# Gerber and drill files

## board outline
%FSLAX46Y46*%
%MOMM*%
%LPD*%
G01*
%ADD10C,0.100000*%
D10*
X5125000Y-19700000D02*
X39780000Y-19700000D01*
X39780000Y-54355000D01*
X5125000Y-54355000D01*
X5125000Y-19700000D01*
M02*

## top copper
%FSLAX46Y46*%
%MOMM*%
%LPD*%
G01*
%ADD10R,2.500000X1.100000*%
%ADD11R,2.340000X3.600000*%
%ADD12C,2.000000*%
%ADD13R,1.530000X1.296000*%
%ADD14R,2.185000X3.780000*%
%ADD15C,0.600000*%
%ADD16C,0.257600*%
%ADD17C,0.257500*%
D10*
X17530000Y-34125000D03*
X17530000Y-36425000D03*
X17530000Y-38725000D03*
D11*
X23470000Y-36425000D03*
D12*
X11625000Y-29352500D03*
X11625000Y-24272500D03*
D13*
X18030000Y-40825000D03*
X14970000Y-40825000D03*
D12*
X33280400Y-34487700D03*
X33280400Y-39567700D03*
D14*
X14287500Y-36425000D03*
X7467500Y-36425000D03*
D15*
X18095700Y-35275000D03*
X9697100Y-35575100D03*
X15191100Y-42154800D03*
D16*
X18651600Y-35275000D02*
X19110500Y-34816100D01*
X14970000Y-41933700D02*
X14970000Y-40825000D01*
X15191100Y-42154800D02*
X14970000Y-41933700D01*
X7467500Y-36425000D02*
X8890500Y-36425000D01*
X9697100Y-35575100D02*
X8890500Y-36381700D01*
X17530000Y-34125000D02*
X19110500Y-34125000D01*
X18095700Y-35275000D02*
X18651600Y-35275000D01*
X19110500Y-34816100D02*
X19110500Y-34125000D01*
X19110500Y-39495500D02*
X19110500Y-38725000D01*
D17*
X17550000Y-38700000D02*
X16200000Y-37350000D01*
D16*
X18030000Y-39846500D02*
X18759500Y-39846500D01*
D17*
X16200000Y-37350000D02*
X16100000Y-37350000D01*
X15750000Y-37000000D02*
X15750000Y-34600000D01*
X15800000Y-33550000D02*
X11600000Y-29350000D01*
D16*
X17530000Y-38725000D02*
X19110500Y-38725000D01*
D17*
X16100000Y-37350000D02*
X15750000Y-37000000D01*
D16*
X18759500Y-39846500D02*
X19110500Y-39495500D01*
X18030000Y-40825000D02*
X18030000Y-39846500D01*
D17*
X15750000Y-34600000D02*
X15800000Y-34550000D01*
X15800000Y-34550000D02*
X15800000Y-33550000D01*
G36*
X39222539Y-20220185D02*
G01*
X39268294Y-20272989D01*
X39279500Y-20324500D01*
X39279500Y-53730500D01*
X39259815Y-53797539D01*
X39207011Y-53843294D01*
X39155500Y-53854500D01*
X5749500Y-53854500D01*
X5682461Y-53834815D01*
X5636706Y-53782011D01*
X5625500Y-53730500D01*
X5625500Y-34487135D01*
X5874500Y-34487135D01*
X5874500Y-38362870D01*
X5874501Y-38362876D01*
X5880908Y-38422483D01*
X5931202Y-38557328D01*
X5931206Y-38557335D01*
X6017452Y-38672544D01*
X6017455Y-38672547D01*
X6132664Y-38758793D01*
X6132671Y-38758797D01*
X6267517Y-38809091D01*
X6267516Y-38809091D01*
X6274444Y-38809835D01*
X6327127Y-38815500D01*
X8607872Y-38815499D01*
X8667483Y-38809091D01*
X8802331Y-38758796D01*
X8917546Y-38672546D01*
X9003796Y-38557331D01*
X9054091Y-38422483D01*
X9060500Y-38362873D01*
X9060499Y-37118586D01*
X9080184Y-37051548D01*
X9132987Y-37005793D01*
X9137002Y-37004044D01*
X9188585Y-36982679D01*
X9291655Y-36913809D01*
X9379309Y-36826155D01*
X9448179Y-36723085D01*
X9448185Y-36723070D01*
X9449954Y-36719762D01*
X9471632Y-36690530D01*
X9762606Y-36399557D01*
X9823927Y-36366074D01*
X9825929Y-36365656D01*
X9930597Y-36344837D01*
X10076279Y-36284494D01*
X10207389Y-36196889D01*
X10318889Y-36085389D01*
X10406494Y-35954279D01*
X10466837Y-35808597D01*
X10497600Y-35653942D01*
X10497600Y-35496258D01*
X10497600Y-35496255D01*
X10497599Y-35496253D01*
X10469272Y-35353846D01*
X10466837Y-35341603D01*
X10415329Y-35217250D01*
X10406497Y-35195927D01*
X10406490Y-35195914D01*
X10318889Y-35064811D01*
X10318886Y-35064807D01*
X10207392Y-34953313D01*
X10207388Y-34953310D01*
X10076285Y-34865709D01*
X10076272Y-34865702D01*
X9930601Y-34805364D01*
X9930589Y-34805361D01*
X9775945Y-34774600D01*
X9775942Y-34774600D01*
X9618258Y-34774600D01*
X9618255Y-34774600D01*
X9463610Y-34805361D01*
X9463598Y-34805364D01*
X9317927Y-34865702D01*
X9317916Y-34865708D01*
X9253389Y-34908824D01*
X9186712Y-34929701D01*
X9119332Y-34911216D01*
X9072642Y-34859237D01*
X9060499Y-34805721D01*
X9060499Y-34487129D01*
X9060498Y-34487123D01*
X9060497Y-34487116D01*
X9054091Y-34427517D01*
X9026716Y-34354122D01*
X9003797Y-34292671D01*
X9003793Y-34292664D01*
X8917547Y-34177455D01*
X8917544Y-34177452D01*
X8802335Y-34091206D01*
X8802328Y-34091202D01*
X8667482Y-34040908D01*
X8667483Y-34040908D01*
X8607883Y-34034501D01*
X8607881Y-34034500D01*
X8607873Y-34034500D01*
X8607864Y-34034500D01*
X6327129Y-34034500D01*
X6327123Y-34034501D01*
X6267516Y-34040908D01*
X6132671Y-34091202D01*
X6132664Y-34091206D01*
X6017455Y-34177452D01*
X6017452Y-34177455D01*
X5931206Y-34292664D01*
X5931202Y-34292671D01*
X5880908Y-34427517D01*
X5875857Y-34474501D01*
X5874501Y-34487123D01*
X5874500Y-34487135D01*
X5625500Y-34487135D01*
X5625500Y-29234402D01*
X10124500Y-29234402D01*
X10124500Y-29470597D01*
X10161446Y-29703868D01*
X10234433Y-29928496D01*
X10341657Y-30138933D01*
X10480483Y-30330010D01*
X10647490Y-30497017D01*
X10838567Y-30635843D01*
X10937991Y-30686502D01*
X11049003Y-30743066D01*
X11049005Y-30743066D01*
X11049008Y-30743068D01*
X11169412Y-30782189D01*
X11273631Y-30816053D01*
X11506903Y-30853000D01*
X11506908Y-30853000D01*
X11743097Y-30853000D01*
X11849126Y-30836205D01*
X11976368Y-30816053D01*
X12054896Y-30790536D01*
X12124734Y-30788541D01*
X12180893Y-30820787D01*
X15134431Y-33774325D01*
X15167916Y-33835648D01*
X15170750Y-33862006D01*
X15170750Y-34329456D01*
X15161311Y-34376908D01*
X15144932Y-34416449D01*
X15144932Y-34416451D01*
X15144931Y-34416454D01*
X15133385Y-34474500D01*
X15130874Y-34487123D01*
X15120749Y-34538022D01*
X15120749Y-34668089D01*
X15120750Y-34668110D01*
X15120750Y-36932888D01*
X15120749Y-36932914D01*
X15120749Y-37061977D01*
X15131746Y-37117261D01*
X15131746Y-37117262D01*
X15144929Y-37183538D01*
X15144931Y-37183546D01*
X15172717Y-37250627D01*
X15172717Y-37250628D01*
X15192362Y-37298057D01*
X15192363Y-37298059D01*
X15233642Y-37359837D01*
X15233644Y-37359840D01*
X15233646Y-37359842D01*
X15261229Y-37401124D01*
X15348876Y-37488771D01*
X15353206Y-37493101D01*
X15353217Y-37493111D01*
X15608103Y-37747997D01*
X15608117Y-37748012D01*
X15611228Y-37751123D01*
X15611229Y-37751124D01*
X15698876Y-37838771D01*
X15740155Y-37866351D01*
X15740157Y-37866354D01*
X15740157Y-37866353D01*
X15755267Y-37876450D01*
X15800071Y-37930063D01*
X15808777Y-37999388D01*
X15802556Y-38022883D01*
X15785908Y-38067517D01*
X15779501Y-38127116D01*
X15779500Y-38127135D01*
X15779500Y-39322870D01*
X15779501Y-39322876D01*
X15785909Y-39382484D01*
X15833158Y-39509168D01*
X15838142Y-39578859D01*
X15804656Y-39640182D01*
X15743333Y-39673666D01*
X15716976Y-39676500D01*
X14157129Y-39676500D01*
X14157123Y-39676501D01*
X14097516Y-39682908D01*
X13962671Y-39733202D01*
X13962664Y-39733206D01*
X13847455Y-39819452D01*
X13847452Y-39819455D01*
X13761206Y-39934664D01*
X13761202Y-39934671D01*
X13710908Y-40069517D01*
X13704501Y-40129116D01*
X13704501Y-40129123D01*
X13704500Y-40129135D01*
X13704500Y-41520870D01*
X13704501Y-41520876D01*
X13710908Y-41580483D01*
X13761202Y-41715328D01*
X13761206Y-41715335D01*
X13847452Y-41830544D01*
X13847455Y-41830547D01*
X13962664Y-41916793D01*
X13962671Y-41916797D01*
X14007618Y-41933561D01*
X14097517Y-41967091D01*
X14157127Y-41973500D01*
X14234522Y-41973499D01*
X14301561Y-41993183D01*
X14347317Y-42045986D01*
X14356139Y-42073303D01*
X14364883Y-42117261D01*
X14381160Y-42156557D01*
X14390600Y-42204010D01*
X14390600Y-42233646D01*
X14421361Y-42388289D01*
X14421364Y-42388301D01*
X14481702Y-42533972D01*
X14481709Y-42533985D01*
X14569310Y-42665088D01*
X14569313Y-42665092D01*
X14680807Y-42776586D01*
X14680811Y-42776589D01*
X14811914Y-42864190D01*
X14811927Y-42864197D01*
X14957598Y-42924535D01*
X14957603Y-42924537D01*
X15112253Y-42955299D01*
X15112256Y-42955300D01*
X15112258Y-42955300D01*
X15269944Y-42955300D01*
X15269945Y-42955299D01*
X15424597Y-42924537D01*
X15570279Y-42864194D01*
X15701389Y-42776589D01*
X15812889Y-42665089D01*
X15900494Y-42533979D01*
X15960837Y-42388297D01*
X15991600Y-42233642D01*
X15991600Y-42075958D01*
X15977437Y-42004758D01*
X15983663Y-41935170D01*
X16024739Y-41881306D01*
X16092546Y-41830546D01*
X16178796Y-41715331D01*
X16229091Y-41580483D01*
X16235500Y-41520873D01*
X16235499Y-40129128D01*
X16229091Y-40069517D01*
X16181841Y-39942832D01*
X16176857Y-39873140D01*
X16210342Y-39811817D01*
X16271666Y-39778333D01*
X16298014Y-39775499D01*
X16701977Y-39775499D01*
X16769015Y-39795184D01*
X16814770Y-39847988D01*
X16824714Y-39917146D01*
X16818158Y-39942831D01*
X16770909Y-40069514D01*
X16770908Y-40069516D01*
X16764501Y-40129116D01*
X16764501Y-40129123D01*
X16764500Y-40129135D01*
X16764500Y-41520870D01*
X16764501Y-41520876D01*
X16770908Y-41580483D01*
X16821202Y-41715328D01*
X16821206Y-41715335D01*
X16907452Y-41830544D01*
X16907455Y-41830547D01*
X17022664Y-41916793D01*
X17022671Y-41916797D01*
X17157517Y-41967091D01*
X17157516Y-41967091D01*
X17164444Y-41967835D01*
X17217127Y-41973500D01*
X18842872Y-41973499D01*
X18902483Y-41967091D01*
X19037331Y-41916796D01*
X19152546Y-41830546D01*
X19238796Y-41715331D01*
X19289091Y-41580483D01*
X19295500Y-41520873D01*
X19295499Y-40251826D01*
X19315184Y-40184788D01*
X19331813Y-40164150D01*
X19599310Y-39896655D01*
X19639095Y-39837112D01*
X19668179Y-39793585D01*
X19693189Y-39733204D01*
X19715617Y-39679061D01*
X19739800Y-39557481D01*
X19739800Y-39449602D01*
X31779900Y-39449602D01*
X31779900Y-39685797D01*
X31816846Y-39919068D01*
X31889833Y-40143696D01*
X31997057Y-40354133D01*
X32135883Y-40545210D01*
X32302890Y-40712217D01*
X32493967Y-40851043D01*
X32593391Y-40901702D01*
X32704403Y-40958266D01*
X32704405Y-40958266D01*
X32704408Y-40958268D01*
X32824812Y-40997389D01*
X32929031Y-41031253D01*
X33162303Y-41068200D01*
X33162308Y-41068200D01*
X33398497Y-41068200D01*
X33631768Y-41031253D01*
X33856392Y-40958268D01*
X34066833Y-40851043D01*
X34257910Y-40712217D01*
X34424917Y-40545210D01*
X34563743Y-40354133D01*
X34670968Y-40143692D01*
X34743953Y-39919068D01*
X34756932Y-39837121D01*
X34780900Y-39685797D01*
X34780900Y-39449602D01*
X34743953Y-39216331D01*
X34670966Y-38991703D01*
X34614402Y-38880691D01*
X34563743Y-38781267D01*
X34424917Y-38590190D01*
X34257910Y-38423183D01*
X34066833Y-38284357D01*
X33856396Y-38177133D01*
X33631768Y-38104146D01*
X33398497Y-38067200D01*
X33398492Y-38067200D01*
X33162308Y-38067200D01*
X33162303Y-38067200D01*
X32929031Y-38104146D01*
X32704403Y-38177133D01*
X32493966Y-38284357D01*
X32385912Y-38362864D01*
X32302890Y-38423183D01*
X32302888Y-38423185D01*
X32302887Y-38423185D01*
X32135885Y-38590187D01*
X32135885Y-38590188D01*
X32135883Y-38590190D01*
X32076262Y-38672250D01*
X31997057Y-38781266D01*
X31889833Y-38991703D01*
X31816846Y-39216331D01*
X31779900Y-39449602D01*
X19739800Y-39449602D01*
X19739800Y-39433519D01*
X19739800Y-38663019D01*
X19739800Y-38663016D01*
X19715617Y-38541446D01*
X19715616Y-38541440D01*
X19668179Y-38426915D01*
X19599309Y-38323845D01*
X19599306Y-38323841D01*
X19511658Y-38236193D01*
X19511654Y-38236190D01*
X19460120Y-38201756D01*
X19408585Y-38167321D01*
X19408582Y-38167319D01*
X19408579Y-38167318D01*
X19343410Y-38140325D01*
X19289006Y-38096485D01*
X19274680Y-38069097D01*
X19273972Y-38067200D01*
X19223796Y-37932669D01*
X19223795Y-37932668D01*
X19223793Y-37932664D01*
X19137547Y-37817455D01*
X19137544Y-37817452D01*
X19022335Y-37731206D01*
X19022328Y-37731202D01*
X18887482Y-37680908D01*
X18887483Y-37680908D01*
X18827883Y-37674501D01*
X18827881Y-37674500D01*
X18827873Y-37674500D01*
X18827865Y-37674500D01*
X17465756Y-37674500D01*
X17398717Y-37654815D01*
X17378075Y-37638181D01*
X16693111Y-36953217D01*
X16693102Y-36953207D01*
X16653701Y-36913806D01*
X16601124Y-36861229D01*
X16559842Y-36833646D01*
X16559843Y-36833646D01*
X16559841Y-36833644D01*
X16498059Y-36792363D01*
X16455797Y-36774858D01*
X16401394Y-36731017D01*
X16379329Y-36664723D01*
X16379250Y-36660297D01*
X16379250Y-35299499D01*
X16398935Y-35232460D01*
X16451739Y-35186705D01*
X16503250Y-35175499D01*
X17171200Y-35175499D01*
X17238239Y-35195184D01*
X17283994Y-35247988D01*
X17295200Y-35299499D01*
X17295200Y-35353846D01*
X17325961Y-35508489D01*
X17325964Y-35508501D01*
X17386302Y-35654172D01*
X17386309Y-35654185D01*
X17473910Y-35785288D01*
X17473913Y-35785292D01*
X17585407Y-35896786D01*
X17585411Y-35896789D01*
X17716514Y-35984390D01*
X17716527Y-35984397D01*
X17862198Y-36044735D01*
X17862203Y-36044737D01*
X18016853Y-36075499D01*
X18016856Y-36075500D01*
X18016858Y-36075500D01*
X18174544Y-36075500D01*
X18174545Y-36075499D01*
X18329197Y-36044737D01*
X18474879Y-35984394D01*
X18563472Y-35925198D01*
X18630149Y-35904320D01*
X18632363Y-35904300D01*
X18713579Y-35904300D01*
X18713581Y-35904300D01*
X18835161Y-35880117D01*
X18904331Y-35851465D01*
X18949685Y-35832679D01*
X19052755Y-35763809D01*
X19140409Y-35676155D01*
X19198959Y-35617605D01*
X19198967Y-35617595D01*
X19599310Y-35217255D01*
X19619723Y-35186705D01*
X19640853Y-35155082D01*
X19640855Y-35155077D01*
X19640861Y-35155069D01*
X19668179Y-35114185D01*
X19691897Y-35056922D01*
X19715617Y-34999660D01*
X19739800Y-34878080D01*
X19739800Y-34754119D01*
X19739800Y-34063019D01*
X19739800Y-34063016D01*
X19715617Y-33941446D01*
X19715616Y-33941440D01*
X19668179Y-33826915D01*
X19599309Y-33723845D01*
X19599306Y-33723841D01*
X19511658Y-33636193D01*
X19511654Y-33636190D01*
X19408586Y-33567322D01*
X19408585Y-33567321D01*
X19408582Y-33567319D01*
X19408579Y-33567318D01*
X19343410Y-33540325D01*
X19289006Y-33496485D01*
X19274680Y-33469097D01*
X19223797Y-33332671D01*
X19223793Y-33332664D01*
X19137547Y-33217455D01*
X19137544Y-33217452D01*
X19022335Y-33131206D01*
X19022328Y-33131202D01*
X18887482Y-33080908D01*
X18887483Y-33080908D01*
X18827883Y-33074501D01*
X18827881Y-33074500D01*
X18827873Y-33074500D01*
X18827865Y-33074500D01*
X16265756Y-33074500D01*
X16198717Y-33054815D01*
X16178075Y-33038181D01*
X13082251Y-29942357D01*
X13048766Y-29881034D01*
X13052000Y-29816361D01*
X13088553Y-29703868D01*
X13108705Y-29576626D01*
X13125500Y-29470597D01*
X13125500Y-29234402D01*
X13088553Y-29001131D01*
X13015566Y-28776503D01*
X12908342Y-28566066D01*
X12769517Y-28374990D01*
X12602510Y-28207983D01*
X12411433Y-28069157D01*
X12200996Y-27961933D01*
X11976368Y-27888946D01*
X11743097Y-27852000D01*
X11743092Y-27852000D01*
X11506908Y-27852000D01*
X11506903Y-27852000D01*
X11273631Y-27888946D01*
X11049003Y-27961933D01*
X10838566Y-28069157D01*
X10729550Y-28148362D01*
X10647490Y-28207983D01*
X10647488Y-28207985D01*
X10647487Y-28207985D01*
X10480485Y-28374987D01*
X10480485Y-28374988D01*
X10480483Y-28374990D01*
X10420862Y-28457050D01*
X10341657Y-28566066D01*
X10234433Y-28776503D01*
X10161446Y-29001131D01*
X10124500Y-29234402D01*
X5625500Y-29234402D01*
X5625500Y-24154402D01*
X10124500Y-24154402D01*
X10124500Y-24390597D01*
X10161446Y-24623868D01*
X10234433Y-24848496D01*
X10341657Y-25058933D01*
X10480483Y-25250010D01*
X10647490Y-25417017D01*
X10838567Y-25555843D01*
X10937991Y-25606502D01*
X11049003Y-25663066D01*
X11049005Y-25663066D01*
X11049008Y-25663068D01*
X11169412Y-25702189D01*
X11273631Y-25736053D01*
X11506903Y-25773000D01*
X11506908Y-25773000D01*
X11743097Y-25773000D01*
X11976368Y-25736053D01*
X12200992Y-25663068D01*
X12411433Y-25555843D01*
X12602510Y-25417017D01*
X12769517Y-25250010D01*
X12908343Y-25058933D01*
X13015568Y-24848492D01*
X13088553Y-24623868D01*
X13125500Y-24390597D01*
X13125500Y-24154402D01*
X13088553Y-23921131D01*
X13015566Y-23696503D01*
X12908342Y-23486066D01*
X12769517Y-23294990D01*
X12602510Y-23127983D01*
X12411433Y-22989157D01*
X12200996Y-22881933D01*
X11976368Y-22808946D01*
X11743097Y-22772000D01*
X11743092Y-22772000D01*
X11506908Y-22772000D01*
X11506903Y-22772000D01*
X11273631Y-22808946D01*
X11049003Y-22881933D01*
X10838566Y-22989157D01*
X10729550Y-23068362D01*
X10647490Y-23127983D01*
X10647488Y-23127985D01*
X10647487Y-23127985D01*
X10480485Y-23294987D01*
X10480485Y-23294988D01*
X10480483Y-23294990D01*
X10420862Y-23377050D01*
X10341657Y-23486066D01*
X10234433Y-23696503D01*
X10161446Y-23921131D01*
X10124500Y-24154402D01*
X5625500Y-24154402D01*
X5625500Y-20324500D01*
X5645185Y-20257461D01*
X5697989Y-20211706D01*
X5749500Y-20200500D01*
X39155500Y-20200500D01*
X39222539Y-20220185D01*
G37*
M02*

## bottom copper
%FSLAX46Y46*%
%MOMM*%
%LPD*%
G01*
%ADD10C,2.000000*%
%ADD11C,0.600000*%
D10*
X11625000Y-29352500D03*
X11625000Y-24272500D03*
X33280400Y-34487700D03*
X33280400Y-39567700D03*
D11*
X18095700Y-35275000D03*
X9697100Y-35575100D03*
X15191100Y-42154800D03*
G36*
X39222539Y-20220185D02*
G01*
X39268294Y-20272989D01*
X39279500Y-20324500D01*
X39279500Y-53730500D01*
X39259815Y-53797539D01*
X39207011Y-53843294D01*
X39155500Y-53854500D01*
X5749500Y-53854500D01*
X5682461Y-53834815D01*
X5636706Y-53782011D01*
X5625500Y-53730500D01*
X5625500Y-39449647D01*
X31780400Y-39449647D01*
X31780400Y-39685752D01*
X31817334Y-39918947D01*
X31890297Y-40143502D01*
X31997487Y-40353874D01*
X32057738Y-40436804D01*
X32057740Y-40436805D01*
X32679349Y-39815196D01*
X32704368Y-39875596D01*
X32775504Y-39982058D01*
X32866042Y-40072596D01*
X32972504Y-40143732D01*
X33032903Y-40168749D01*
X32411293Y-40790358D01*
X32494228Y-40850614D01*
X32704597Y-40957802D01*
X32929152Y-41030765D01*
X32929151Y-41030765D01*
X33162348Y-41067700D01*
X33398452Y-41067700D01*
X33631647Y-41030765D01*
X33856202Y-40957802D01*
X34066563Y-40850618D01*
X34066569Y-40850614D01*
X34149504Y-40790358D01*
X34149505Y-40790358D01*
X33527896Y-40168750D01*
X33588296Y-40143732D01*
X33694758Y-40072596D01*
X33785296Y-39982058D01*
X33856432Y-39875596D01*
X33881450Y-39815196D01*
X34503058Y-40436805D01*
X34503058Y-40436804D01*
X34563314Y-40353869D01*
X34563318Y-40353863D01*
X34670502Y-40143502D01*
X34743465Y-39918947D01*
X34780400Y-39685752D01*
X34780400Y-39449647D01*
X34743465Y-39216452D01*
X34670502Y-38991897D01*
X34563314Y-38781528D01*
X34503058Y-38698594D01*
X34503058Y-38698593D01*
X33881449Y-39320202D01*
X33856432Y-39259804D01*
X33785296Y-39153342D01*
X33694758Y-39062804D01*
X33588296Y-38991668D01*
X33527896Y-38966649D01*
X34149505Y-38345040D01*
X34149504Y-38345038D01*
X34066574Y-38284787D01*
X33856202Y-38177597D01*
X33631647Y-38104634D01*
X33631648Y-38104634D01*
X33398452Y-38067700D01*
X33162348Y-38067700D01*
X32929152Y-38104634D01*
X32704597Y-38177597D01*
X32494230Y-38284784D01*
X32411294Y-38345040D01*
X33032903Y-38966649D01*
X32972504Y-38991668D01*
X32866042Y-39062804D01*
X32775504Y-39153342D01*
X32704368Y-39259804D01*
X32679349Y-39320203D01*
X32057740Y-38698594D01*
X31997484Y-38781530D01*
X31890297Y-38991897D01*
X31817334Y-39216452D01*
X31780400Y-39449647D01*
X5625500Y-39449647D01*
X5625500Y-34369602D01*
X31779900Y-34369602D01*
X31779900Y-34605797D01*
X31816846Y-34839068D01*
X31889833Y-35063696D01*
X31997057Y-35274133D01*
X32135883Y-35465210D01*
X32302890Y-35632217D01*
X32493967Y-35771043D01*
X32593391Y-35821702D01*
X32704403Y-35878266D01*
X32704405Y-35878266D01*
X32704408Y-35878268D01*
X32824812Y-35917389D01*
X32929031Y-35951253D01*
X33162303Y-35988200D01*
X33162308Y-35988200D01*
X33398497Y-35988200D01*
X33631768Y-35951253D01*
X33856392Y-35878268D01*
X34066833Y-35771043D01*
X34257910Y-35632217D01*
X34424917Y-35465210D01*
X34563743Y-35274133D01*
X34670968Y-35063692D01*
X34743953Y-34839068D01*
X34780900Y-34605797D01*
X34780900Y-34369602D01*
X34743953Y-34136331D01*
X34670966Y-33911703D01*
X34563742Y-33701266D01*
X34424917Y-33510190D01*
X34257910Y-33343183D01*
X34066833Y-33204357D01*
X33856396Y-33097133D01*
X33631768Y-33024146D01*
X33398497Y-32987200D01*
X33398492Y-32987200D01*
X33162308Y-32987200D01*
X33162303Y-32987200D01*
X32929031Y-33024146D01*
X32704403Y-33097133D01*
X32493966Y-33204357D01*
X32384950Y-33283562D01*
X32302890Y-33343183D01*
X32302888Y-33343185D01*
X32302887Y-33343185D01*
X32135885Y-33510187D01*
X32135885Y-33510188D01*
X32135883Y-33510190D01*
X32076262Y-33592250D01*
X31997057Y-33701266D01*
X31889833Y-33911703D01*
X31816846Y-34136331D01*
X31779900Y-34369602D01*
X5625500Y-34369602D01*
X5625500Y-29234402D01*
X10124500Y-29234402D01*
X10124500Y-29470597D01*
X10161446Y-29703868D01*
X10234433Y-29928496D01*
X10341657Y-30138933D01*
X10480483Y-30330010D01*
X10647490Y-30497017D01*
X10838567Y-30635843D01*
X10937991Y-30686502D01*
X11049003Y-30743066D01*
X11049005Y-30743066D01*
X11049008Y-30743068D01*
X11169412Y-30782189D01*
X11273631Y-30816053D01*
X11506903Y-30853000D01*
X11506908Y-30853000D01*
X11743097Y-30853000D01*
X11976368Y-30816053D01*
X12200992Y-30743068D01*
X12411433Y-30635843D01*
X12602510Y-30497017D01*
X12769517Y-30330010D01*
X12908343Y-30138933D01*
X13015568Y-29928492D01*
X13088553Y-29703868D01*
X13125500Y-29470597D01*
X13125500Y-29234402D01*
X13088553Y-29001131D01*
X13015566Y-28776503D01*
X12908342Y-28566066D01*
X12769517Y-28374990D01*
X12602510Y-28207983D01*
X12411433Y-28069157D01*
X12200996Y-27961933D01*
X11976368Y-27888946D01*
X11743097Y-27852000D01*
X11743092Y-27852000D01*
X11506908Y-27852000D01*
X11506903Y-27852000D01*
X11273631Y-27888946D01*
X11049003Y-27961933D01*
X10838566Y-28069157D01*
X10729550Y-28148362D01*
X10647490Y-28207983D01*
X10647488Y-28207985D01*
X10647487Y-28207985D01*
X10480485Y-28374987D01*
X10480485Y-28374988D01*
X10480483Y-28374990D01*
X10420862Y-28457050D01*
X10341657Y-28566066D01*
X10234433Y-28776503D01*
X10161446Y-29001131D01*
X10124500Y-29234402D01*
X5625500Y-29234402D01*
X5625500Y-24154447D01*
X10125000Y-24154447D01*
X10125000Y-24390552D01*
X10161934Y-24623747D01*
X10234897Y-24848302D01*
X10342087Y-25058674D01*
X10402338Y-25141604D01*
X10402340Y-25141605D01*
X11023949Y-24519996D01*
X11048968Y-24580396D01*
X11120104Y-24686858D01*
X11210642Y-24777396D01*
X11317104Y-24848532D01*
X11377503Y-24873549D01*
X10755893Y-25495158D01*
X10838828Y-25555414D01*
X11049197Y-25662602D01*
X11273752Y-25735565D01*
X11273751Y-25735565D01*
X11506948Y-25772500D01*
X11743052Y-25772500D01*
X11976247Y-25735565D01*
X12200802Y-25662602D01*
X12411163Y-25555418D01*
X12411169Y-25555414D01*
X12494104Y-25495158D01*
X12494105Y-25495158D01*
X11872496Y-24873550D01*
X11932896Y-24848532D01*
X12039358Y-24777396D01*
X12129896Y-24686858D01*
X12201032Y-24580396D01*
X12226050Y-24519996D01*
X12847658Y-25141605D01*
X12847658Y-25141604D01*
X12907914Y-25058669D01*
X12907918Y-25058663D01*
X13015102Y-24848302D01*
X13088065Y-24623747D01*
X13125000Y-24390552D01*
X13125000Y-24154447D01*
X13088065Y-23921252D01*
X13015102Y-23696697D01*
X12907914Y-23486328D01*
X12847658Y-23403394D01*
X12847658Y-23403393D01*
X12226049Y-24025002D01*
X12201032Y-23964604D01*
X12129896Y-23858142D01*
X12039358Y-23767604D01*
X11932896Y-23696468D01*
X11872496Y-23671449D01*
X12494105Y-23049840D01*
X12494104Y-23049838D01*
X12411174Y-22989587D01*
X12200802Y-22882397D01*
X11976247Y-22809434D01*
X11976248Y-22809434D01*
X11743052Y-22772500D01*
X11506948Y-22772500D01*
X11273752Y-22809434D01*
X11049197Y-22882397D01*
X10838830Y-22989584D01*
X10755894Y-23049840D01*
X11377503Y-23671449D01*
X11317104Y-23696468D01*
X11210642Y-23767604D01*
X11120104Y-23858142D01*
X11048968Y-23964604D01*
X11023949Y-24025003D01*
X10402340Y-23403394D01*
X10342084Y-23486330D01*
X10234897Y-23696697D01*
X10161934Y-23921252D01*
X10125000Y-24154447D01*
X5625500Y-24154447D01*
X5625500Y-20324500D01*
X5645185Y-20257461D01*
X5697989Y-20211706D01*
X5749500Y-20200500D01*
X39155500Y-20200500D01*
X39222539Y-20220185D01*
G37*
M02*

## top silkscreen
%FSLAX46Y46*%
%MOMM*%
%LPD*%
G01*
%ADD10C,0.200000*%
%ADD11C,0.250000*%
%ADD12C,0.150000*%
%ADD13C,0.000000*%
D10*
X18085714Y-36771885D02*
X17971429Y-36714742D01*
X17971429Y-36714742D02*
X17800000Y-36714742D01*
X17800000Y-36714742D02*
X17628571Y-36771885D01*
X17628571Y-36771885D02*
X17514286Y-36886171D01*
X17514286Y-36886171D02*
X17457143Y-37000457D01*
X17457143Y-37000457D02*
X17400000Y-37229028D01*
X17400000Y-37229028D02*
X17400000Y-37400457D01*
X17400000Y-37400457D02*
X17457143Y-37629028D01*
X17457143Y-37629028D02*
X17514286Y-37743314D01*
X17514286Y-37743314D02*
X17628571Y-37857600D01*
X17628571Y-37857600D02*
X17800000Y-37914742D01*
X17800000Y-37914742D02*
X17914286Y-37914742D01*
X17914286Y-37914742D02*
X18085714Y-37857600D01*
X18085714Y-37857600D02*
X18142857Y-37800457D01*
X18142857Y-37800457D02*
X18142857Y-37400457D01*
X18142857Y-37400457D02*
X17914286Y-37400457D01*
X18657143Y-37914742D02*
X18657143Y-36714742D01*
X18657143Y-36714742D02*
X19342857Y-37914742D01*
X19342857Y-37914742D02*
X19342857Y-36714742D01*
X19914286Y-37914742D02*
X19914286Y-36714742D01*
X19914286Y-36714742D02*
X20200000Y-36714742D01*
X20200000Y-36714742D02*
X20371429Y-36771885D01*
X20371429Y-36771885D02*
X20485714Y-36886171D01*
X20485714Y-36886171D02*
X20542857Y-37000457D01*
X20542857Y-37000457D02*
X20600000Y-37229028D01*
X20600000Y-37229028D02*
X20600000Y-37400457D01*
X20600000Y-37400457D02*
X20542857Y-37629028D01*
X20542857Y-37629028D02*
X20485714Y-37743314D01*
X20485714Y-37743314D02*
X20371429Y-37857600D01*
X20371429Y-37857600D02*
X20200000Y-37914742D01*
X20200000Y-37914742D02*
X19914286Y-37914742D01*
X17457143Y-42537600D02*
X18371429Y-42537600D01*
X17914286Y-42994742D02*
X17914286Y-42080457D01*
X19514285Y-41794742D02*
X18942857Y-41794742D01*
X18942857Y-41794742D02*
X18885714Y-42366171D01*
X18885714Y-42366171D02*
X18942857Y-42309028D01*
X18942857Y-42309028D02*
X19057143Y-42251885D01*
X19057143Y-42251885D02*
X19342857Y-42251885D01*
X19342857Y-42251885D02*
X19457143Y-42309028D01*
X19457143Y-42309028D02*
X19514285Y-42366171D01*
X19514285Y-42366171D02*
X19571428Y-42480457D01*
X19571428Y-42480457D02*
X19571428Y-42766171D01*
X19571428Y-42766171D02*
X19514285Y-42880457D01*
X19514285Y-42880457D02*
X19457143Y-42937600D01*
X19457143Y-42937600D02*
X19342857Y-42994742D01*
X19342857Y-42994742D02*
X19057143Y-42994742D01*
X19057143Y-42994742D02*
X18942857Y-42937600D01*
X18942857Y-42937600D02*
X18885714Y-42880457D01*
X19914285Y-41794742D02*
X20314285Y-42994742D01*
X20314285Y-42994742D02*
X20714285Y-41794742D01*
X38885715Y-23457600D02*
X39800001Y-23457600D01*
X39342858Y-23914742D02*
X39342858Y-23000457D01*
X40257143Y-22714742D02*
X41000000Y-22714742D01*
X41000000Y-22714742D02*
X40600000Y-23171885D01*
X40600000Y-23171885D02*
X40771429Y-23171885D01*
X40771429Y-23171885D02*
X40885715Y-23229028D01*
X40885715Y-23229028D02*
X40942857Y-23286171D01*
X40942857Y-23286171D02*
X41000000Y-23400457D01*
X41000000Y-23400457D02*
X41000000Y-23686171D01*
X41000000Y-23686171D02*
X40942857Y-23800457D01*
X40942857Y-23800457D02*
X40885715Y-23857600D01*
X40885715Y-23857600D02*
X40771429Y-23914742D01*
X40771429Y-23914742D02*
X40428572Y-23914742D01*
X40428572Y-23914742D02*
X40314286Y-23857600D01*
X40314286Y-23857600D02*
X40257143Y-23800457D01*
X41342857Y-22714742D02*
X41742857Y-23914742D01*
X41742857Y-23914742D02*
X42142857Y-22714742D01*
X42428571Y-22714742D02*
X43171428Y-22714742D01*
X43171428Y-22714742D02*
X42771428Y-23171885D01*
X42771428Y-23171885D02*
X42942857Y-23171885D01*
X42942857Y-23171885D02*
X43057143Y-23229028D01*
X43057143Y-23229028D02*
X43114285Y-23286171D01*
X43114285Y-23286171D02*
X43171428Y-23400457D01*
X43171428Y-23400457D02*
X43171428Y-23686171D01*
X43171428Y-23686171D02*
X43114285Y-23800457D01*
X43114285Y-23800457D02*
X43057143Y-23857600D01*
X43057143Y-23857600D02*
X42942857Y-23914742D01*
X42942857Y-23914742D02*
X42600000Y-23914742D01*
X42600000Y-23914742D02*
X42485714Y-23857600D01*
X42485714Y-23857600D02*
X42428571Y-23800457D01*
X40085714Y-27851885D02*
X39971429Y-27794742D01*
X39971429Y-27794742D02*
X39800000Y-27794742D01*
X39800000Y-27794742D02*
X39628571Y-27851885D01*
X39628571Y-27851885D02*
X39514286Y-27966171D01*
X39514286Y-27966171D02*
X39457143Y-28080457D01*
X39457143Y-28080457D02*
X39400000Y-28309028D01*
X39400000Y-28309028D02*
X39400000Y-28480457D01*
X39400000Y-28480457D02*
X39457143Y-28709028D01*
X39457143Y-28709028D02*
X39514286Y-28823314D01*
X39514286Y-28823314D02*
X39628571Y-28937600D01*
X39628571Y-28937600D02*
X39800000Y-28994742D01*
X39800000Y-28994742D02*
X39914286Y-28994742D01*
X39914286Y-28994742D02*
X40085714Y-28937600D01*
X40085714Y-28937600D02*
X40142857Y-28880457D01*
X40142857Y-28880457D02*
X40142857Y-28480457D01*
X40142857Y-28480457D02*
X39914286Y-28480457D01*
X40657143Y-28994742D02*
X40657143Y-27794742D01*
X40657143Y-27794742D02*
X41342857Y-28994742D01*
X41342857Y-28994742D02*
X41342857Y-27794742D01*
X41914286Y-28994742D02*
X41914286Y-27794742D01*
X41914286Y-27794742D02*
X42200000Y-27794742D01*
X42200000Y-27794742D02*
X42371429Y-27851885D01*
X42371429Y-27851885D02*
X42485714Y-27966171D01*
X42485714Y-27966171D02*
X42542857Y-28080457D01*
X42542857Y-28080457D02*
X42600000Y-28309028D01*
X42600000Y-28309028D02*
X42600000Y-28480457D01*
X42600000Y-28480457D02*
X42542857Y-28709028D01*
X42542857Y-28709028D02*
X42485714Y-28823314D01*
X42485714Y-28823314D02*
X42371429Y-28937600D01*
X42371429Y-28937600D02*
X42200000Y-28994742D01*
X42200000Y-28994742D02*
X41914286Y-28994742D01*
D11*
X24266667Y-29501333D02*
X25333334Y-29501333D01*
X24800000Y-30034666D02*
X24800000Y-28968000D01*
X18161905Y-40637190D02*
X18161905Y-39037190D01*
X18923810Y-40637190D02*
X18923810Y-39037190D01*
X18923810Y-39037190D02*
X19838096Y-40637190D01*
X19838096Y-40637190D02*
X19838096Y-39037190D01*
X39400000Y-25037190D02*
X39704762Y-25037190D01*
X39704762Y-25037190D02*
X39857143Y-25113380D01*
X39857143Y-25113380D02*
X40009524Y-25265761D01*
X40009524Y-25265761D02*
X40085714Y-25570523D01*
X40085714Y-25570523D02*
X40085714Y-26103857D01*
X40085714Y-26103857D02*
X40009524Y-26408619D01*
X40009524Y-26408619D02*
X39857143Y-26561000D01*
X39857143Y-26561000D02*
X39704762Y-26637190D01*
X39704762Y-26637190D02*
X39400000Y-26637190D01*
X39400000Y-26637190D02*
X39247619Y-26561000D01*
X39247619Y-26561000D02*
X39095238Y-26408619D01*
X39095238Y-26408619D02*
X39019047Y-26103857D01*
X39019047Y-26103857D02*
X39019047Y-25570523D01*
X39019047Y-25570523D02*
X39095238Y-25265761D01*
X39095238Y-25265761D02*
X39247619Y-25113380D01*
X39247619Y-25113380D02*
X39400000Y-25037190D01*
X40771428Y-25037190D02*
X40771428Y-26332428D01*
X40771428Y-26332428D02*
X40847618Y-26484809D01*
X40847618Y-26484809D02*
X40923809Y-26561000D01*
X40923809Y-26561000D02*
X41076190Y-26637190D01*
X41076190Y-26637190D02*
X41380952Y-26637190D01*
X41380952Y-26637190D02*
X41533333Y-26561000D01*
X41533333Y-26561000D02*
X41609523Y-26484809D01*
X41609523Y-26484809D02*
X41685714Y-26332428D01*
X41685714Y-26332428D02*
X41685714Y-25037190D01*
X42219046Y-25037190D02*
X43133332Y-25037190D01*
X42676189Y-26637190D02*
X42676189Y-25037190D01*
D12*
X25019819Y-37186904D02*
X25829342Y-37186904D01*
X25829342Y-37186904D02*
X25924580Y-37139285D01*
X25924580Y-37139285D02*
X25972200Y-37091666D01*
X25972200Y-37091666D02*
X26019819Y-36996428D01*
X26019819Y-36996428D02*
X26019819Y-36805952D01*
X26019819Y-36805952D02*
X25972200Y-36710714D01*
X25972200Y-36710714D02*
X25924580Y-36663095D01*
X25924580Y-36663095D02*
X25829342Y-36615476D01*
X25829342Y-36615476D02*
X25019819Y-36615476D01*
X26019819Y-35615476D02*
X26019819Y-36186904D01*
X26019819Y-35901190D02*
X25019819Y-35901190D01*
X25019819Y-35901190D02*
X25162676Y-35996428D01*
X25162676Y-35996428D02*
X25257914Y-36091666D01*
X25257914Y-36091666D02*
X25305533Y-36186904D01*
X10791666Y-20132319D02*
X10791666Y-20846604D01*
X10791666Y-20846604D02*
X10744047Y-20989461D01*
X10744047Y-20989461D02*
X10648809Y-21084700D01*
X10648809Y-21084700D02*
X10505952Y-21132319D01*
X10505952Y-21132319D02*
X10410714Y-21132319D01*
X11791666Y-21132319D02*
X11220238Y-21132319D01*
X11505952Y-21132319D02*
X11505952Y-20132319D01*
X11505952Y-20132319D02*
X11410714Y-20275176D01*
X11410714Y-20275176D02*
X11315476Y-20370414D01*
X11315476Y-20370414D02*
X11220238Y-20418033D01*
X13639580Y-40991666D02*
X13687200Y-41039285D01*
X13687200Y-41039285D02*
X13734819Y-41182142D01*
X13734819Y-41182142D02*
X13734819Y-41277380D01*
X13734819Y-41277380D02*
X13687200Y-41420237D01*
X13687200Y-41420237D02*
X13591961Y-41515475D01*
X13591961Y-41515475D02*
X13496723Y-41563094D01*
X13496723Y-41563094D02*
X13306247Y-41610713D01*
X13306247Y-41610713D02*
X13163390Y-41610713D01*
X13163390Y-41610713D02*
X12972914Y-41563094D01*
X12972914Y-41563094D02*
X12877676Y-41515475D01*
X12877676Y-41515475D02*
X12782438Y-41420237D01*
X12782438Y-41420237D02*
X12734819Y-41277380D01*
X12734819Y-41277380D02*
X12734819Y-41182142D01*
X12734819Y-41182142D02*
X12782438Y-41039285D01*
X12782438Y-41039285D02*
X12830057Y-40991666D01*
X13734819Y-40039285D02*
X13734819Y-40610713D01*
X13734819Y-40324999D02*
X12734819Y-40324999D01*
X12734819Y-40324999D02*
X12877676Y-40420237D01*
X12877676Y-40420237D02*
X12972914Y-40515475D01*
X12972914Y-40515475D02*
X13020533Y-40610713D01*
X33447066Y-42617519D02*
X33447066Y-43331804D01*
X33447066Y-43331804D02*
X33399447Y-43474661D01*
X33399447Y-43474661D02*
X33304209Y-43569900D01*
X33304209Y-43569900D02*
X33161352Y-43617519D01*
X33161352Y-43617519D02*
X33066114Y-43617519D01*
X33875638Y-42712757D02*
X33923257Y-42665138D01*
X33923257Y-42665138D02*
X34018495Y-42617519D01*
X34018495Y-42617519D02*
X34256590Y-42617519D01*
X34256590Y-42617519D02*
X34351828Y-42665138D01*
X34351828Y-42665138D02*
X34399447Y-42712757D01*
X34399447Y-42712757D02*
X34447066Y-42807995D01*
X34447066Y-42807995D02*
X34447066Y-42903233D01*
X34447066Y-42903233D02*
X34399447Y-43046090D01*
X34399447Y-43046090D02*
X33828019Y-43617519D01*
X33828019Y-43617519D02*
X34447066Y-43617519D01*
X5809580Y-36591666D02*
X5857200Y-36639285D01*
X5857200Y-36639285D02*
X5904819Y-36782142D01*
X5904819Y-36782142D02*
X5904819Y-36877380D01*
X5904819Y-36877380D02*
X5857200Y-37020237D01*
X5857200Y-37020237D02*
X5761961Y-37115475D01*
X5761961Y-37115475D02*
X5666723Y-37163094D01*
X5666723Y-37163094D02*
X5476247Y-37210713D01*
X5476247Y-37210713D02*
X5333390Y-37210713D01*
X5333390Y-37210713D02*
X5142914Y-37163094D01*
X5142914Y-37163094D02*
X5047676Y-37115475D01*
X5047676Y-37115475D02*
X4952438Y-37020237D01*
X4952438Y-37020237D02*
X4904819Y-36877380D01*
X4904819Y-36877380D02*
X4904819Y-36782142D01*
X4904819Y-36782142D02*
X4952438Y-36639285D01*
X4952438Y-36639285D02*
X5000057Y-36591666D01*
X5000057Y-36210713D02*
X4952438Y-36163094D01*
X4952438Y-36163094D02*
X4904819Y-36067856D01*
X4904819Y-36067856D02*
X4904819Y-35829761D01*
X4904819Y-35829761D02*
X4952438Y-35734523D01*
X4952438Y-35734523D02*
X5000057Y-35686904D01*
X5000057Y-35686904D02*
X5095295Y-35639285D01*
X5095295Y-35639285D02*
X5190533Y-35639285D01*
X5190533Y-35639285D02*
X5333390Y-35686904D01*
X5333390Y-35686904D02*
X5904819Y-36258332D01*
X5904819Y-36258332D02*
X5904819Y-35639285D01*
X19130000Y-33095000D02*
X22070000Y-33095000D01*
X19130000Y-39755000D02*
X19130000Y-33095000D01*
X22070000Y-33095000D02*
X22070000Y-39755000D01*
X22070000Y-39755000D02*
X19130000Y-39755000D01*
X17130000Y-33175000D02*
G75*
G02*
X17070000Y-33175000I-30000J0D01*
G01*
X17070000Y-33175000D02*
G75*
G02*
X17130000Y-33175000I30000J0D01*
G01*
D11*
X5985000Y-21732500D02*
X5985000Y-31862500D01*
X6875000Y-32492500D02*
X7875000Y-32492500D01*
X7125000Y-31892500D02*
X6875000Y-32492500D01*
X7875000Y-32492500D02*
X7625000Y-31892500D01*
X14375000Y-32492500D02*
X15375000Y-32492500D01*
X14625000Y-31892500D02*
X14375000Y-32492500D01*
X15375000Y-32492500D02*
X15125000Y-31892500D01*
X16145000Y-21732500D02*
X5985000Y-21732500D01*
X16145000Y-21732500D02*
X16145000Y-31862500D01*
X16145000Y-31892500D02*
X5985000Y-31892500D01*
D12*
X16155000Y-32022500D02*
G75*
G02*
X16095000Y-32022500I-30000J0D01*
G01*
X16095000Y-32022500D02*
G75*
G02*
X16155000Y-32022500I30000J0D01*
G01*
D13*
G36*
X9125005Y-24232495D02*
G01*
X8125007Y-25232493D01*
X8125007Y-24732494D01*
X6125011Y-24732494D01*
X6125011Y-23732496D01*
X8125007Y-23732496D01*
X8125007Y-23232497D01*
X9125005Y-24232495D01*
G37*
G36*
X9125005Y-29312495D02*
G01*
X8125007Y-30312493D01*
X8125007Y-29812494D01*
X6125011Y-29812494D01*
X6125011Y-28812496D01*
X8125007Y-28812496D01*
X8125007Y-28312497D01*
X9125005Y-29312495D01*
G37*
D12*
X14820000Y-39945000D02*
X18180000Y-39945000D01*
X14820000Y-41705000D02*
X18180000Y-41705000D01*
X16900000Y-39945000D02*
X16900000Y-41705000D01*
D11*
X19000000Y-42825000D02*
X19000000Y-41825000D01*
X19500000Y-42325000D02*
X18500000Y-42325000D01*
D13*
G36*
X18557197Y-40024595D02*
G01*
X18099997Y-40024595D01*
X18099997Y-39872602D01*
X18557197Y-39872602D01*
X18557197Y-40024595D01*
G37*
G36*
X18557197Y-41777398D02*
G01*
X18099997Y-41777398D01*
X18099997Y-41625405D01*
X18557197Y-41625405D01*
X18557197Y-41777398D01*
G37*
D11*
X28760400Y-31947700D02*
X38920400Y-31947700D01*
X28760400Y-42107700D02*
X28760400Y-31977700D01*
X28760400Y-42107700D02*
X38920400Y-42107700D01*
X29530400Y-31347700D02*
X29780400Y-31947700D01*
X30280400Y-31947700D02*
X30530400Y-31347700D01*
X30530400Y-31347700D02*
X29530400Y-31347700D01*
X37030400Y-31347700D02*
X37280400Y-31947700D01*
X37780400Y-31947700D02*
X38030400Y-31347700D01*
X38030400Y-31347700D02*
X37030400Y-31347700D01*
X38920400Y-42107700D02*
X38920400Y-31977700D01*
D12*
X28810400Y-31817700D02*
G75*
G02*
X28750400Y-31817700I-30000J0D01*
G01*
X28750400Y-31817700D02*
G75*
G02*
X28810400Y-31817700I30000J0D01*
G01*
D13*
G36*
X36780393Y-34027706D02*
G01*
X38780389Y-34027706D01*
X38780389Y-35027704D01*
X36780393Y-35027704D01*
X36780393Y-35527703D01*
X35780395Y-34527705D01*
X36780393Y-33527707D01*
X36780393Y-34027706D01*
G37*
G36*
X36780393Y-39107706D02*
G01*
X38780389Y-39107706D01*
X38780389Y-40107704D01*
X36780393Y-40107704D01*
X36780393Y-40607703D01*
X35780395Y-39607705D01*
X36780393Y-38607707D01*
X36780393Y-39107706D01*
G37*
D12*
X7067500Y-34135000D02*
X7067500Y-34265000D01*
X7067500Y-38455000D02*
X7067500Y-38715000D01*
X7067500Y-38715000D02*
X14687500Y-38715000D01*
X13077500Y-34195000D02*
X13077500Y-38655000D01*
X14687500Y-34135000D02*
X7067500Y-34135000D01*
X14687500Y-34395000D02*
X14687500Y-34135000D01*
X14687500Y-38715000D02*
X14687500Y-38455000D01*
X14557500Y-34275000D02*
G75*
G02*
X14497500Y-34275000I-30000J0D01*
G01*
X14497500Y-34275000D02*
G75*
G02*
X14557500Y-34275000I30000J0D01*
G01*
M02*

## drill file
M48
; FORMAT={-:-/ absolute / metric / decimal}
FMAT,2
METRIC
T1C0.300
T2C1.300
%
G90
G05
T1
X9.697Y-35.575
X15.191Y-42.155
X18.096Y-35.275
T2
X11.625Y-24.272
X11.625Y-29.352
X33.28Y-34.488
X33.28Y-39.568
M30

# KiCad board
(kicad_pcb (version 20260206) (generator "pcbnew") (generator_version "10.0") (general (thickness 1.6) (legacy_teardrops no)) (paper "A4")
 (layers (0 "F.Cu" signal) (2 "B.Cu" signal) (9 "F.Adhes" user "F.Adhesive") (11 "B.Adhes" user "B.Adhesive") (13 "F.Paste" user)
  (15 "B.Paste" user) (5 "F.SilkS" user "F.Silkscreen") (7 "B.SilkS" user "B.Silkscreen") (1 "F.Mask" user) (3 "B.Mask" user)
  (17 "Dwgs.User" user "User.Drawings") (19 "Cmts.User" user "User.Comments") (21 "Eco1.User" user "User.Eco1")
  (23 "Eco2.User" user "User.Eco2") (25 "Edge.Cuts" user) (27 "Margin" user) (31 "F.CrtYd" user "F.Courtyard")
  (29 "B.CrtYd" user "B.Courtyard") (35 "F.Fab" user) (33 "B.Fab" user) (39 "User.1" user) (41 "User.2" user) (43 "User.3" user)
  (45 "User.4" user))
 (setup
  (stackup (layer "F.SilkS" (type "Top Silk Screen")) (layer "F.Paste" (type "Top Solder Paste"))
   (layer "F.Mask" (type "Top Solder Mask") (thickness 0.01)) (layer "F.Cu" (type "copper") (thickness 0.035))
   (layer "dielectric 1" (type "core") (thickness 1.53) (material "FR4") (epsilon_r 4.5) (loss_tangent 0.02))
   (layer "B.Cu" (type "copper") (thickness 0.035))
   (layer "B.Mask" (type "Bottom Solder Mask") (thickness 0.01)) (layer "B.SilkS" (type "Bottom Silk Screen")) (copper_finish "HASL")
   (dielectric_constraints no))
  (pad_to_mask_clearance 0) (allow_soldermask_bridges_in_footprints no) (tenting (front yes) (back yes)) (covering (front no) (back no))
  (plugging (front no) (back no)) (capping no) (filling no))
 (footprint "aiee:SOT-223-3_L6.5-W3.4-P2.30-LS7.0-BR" (layer "F.Cu") (at 20.5 36.425 180)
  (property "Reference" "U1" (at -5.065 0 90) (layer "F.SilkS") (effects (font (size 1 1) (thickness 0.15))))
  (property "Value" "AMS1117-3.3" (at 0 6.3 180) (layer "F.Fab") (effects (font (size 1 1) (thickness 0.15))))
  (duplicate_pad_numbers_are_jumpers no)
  (fp_line (start 1.37 3.33) (end -1.57 3.33) (stroke (width 0.15) (type solid)) (layer "F.SilkS"))
  (fp_line (start 1.37 -3.33) (end 1.37 3.33) (stroke (width 0.15) (type solid)) (layer "F.SilkS"))
  (fp_line (start -1.57 3.33) (end -1.57 -3.33) (stroke (width 0.15) (type solid)) (layer "F.SilkS"))
  (fp_line (start -1.57 -3.33) (end 1.37 -3.33) (stroke (width 0.15) (type solid)) (layer "F.SilkS"))
  (fp_circle (center 3.4 3.25) (end 3.43 3.25) (stroke (width 0.15) (type solid)) (fill no) (layer "F.SilkS"))
  (pad "1" smd rect (at 2.97 2.3 180) (size 2.5 1.1) (layers "F.Cu" "F.Mask" "F.Paste") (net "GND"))
  (pad "2" smd rect (at 2.97 0 180) (size 2.5 1.1) (layers "F.Cu" "F.Mask" "F.Paste") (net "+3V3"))
  (pad "3" smd rect (at 2.97 -2.3 180) (size 2.5 1.1) (layers "F.Cu" "F.Mask" "F.Paste") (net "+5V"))
  (pad "4" smd rect (at -2.97 0 180) (size 2.34 3.6) (layers "F.Cu" "F.Mask" "F.Paste") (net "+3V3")))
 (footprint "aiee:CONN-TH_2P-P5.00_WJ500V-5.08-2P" (layer "F.Cu") (at 11.625 26.8125 90)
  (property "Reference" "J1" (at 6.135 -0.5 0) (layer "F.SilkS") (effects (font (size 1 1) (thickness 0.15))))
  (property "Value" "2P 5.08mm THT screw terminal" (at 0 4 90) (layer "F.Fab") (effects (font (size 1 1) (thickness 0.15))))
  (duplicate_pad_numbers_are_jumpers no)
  (fp_line (start 5.08 -5.64) (end -5.05 -5.64) (stroke (width 0.25) (type solid)) (layer "F.SilkS"))
  (fp_line (start -5.68 -4.75) (end -5.68 -3.75) (stroke (width 0.25) (type solid)) (layer "F.SilkS"))
  (fp_line (start -5.08 -4.5) (end -5.68 -4.75) (stroke (width 0.25) (type solid)) (layer "F.SilkS"))
  (fp_line (start -5.68 -3.75) (end -5.08 -4) (stroke (width 0.25) (type solid)) (layer "F.SilkS"))
  (fp_line (start -5.68 2.75) (end -5.68 3.75) (stroke (width 0.25) (type solid)) (layer "F.SilkS"))
  (fp_line (start -5.08 3) (end -5.68 2.75) (stroke (width 0.25) (type solid)) (layer "F.SilkS"))
  (fp_line (start -5.68 3.75) (end -5.08 3.5) (stroke (width 0.25) (type solid)) (layer "F.SilkS"))
  (fp_line (start 5.08 4.52) (end 5.08 -5.64) (stroke (width 0.25) (type solid)) (layer "F.SilkS"))
  (fp_line (start 5.08 4.52) (end -5.05 4.52) (stroke (width 0.25) (type solid)) (layer "F.SilkS"))
  (fp_line (start -5.08 4.52) (end -5.08 -5.64) (stroke (width 0.25) (type solid)) (layer "F.SilkS"))
  (fp_circle (center -5.21 4.5) (end -5.18 4.5) (stroke (width 0.15) (type solid)) (fill no) (layer "F.SilkS"))
  (fp_poly
   (pts (xy 2.080006 -5.499989) (xy 3.080004 -5.499989) (xy 3.080004 -3.499993) (xy 3.580003 -3.499993) (xy 2.580005 -2.499995)
    (xy 1.580007 -3.499993) (xy 2.080006 -3.499993) (xy 2.080006 -5.499989))
   (stroke (width 0) (type solid)) (fill yes) (layer "F.SilkS"))
  (fp_poly
   (pts (xy -2.999994 -5.499989) (xy -1.999996 -5.499989) (xy -1.999996 -3.499993) (xy -1.499997 -3.499993) (xy -2.499995 -2.499995)
    (xy -3.499993 -3.499993) (xy -2.999994 -3.499993) (xy -2.999994 -5.499989))
   (stroke (width 0) (type solid)) (fill yes) (layer "F.SilkS"))
  (pad "1" thru_hole circle (at -2.54 0 270) (size 2 2) (drill 1.300022) (layers "*.Cu" "*.Mask") (remove_unused_layers no) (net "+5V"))
  (pad "2" thru_hole circle (at 2.54 0 270) (size 2 2) (drill 1.300022) (layers "*.Cu" "*.Mask") (remove_unused_layers no) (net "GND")))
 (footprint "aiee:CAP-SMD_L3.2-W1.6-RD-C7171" (layer "F.Cu") (at 16.5 40.825 180)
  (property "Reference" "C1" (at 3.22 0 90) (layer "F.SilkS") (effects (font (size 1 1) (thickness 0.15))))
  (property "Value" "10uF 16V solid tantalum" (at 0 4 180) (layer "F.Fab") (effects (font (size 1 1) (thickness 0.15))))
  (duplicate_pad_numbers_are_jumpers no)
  (fp_line (start 1.68 0.88) (end -1.68 0.88) (stroke (width 0.15) (type solid)) (layer "F.SilkS"))
  (fp_line (start 1.68 -0.88) (end -1.68 -0.88) (stroke (width 0.15) (type solid)) (layer "F.SilkS"))
  (fp_line (start -0.4 0.88) (end -0.4 -0.88) (stroke (width 0.15) (type solid)) (layer "F.SilkS"))
  (fp_line (start -2.5 -2) (end -2.5 -1) (stroke (width 0.25) (type solid)) (layer "F.SilkS"))
  (fp_line (start -3 -1.5) (end -2 -1.5) (stroke (width 0.25) (type solid)) (layer "F.SilkS"))
  (fp_poly
   (pts (xy -1.599997 0.952398) (xy -1.599997 0.800405) (xy -2.057197 0.800405) (xy -2.057197 0.952398) (xy -1.599997 0.952398))
   (stroke (width 0) (type solid)) (fill yes) (layer "F.SilkS"))
  (fp_poly
   (pts (xy -1.599997 -0.952398) (xy -1.599997 -0.800405) (xy -2.057197 -0.800405) (xy -2.057197 -0.952398) (xy -1.599997 -0.952398))
   (stroke (width 0) (type solid)) (fill yes) (layer "F.SilkS"))
  (pad "1" smd rect (at -1.53 0) (size 1.53 1.296) (layers "F.Cu" "F.Mask" "F.Paste") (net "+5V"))
  (pad "2" smd rect (at 1.53 0) (size 1.53 1.296) (layers "F.Cu" "F.Mask" "F.Paste") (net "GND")))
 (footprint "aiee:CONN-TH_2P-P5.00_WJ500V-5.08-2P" (layer "F.Cu") (at 33.2804 37.0277 -90)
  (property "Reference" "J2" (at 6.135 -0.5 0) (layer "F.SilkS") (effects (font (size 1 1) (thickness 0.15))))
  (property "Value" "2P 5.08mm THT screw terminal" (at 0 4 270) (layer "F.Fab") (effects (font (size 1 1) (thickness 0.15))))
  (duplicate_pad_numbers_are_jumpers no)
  (fp_line (start -5.08 4.52) (end -5.08 -5.64) (stroke (width 0.25) (type solid)) (layer "F.SilkS"))
  (fp_line (start 5.08 4.52) (end -5.05 4.52) (stroke (width 0.25) (type solid)) (layer "F.SilkS"))
  (fp_line (start 5.08 4.52) (end 5.08 -5.64) (stroke (width 0.25) (type solid)) (layer "F.SilkS"))
  (fp_line (start -5.68 3.75) (end -5.08 3.5) (stroke (width 0.25) (type solid)) (layer "F.SilkS"))
  (fp_line (start -5.08 3) (end -5.68 2.75) (stroke (width 0.25) (type solid)) (layer "F.SilkS"))
  (fp_line (start -5.68 2.75) (end -5.68 3.75) (stroke (width 0.25) (type solid)) (layer "F.SilkS"))
  (fp_line (start -5.68 -3.75) (end -5.08 -4) (stroke (width 0.25) (type solid)) (layer "F.SilkS"))
  (fp_line (start -5.08 -4.5) (end -5.68 -4.75) (stroke (width 0.25) (type solid)) (layer "F.SilkS"))
  (fp_line (start -5.68 -4.75) (end -5.68 -3.75) (stroke (width 0.25) (type solid)) (layer "F.SilkS"))
  (fp_line (start 5.08 -5.64) (end -5.05 -5.64) (stroke (width 0.25) (type solid)) (layer "F.SilkS"))
  (fp_circle (center -5.21 4.5) (end -5.18 4.5) (stroke (width 0.15) (type solid)) (fill no) (layer "F.SilkS"))
  (fp_poly
   (pts (xy -2.999994 -5.499989) (xy -1.999996 -5.499989) (xy -1.999996 -3.499993) (xy -1.499997 -3.499993) (xy -2.499995 -2.499995)
    (xy -3.499993 -3.499993) (xy -2.999994 -3.499993) (xy -2.999994 -5.499989))
   (stroke (width 0) (type solid)) (fill yes) (layer "F.SilkS"))
  (fp_poly
   (pts (xy 2.080006 -5.499989) (xy 3.080004 -5.499989) (xy 3.080004 -3.499993) (xy 3.580003 -3.499993) (xy 2.580005 -2.499995)
    (xy 1.580007 -3.499993) (xy 2.080006 -3.499993) (xy 2.080006 -5.499989))
   (stroke (width 0) (type solid)) (fill yes) (layer "F.SilkS"))
  (pad "1" thru_hole circle (at -2.54 0 90) (size 2 2) (drill 1.300022) (layers "*.Cu" "*.Mask") (remove_unused_layers no) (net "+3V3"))
  (pad "2" thru_hole circle (at 2.54 0 90) (size 2 2) (drill 1.300022) (layers "*.Cu" "*.Mask") (remove_unused_layers no) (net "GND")))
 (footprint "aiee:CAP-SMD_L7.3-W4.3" (layer "F.Cu") (at 10.8775 36.425)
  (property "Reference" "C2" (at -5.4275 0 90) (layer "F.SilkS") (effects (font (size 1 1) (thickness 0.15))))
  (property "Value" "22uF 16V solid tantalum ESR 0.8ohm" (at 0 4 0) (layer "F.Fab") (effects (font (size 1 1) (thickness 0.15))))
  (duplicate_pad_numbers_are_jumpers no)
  (fp_line (start -3.81 -2.29) (end -3.81 -2.16) (stroke (width 0.15) (type solid)) (layer "F.SilkS"))
  (fp_line (start -3.81 2.03) (end -3.81 2.29) (stroke (width 0.15) (type solid)) (layer "F.SilkS"))
  (fp_line (start -3.81 2.29) (end 3.81 2.29) (stroke (width 0.15) (type solid)) (layer "F.SilkS"))
  (fp_line (start 2.2 -2.23) (end 2.2 2.23) (stroke (width 0.15) (type solid)) (layer "F.SilkS"))
  (fp_line (start 3.81 -2.29) (end -3.81 -2.29) (stroke (width 0.15) (type solid)) (layer "F.SilkS"))
  (fp_line (start 3.81 -2.03) (end 3.81 -2.29) (stroke (width 0.15) (type solid)) (layer "F.SilkS"))
  (fp_line (start 3.81 2.29) (end 3.81 2.03) (stroke (width 0.15) (type solid)) (layer "F.SilkS"))
  (fp_circle (center 3.65 -2.15) (end 3.68 -2.15) (stroke (width 0.15) (type solid)) (fill no) (layer "F.SilkS"))
  (pad "1" smd rect (at 3.41 0 180) (size 2.185 3.78) (layers "F.Cu" "F.Mask" "F.Paste") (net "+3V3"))
  (pad "2" smd rect (at -3.41 0 180) (size 2.185 3.78) (layers "F.Cu" "F.Mask" "F.Paste") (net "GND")))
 (gr_rect (start 5.125 19.7) (end 39.78 54.355) (stroke (width 0.1) (type default)) (fill no) (layer "Edge.Cuts"))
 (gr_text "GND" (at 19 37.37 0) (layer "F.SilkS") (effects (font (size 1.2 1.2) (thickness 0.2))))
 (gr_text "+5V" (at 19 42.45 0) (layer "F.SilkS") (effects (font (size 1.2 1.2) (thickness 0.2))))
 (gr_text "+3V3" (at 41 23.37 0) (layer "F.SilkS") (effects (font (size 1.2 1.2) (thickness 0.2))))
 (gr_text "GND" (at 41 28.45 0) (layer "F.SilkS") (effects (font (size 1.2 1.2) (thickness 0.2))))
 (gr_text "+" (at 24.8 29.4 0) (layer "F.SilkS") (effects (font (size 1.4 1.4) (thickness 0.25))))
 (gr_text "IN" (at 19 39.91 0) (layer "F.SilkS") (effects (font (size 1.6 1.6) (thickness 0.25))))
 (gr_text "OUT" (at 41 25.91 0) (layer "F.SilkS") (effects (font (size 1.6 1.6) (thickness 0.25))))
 (segment (start 18.6516 35.275) (end 19.1105 34.8161) (width 0.2576) (layer "F.Cu") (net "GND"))
 (segment (start 14.97 41.9337) (end 14.97 40.825) (width 0.2576) (layer "F.Cu") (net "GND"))
 (segment (start 15.1911 42.1548) (end 14.97 41.9337) (width 0.2576) (layer "F.Cu") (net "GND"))
 (segment (start 7.4675 36.425) (end 8.8905 36.425) (width 0.2576) (layer "F.Cu") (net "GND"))
 (segment (start 9.6971 35.5751) (end 8.8905 36.3817) (width 0.2576) (layer "F.Cu") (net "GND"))
 (segment (start 17.53 34.125) (end 19.1105 34.125) (width 0.2576) (layer "F.Cu") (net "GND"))
 (segment (start 18.0957 35.275) (end 18.6516 35.275) (width 0.2576) (layer "F.Cu") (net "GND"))
 (segment (start 19.1105 34.8161) (end 19.1105 34.125) (width 0.2576) (layer "F.Cu") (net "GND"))
 (via (at 18.0957 35.275) (size 0.6) (drill 0.3) (layers "F.Cu" "B.Cu") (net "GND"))
 (via (at 9.6971 35.5751) (size 0.6) (drill 0.3) (layers "F.Cu" "B.Cu") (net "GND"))
 (via (at 15.1911 42.1548) (size 0.6) (drill 0.3) (layers "F.Cu" "B.Cu") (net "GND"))
 (segment (start 19.1105 39.4955) (end 19.1105 38.725) (width 0.2576) (layer "F.Cu") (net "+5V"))
 (segment (start 17.55 38.7) (end 16.2 37.35) (width 0.2575) (layer "F.Cu") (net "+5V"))
 (segment (start 18.03 39.8465) (end 18.7595 39.8465) (width 0.2576) (layer "F.Cu") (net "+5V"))
 (segment (start 16.2 37.35) (end 16.1 37.35) (width 0.2575) (layer "F.Cu") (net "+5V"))
 (segment (start 15.75 37) (end 15.75 34.6) (width 0.2575) (layer "F.Cu") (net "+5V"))
 (segment (start 15.8 33.55) (end 11.6 29.35) (width 0.2575) (layer "F.Cu") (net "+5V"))
 (segment (start 17.53 38.725) (end 19.1105 38.725) (width 0.2576) (layer "F.Cu") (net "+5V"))
 (segment (start 16.1 37.35) (end 15.75 37) (width 0.2575) (layer "F.Cu") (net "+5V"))
 (segment (start 18.7595 39.8465) (end 19.1105 39.4955) (width 0.2576) (layer "F.Cu") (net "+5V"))
 (segment (start 18.03 40.825) (end 18.03 39.8465) (width 0.2576) (layer "F.Cu") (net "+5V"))
 (segment (start 15.75 34.6) (end 15.8 34.55) (width 0.2575) (layer "F.Cu") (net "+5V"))
 (segment (start 15.8 34.55) (end 15.8 33.55) (width 0.2575) (layer "F.Cu") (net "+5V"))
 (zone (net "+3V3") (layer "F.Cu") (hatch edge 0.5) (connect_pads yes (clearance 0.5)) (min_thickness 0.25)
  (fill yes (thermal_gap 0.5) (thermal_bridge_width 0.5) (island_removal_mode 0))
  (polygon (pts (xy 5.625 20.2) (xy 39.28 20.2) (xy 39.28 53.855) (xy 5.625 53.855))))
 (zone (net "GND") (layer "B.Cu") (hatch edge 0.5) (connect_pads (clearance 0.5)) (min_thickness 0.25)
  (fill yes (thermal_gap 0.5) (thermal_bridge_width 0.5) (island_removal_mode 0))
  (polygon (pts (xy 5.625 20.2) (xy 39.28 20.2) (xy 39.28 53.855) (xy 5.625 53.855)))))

